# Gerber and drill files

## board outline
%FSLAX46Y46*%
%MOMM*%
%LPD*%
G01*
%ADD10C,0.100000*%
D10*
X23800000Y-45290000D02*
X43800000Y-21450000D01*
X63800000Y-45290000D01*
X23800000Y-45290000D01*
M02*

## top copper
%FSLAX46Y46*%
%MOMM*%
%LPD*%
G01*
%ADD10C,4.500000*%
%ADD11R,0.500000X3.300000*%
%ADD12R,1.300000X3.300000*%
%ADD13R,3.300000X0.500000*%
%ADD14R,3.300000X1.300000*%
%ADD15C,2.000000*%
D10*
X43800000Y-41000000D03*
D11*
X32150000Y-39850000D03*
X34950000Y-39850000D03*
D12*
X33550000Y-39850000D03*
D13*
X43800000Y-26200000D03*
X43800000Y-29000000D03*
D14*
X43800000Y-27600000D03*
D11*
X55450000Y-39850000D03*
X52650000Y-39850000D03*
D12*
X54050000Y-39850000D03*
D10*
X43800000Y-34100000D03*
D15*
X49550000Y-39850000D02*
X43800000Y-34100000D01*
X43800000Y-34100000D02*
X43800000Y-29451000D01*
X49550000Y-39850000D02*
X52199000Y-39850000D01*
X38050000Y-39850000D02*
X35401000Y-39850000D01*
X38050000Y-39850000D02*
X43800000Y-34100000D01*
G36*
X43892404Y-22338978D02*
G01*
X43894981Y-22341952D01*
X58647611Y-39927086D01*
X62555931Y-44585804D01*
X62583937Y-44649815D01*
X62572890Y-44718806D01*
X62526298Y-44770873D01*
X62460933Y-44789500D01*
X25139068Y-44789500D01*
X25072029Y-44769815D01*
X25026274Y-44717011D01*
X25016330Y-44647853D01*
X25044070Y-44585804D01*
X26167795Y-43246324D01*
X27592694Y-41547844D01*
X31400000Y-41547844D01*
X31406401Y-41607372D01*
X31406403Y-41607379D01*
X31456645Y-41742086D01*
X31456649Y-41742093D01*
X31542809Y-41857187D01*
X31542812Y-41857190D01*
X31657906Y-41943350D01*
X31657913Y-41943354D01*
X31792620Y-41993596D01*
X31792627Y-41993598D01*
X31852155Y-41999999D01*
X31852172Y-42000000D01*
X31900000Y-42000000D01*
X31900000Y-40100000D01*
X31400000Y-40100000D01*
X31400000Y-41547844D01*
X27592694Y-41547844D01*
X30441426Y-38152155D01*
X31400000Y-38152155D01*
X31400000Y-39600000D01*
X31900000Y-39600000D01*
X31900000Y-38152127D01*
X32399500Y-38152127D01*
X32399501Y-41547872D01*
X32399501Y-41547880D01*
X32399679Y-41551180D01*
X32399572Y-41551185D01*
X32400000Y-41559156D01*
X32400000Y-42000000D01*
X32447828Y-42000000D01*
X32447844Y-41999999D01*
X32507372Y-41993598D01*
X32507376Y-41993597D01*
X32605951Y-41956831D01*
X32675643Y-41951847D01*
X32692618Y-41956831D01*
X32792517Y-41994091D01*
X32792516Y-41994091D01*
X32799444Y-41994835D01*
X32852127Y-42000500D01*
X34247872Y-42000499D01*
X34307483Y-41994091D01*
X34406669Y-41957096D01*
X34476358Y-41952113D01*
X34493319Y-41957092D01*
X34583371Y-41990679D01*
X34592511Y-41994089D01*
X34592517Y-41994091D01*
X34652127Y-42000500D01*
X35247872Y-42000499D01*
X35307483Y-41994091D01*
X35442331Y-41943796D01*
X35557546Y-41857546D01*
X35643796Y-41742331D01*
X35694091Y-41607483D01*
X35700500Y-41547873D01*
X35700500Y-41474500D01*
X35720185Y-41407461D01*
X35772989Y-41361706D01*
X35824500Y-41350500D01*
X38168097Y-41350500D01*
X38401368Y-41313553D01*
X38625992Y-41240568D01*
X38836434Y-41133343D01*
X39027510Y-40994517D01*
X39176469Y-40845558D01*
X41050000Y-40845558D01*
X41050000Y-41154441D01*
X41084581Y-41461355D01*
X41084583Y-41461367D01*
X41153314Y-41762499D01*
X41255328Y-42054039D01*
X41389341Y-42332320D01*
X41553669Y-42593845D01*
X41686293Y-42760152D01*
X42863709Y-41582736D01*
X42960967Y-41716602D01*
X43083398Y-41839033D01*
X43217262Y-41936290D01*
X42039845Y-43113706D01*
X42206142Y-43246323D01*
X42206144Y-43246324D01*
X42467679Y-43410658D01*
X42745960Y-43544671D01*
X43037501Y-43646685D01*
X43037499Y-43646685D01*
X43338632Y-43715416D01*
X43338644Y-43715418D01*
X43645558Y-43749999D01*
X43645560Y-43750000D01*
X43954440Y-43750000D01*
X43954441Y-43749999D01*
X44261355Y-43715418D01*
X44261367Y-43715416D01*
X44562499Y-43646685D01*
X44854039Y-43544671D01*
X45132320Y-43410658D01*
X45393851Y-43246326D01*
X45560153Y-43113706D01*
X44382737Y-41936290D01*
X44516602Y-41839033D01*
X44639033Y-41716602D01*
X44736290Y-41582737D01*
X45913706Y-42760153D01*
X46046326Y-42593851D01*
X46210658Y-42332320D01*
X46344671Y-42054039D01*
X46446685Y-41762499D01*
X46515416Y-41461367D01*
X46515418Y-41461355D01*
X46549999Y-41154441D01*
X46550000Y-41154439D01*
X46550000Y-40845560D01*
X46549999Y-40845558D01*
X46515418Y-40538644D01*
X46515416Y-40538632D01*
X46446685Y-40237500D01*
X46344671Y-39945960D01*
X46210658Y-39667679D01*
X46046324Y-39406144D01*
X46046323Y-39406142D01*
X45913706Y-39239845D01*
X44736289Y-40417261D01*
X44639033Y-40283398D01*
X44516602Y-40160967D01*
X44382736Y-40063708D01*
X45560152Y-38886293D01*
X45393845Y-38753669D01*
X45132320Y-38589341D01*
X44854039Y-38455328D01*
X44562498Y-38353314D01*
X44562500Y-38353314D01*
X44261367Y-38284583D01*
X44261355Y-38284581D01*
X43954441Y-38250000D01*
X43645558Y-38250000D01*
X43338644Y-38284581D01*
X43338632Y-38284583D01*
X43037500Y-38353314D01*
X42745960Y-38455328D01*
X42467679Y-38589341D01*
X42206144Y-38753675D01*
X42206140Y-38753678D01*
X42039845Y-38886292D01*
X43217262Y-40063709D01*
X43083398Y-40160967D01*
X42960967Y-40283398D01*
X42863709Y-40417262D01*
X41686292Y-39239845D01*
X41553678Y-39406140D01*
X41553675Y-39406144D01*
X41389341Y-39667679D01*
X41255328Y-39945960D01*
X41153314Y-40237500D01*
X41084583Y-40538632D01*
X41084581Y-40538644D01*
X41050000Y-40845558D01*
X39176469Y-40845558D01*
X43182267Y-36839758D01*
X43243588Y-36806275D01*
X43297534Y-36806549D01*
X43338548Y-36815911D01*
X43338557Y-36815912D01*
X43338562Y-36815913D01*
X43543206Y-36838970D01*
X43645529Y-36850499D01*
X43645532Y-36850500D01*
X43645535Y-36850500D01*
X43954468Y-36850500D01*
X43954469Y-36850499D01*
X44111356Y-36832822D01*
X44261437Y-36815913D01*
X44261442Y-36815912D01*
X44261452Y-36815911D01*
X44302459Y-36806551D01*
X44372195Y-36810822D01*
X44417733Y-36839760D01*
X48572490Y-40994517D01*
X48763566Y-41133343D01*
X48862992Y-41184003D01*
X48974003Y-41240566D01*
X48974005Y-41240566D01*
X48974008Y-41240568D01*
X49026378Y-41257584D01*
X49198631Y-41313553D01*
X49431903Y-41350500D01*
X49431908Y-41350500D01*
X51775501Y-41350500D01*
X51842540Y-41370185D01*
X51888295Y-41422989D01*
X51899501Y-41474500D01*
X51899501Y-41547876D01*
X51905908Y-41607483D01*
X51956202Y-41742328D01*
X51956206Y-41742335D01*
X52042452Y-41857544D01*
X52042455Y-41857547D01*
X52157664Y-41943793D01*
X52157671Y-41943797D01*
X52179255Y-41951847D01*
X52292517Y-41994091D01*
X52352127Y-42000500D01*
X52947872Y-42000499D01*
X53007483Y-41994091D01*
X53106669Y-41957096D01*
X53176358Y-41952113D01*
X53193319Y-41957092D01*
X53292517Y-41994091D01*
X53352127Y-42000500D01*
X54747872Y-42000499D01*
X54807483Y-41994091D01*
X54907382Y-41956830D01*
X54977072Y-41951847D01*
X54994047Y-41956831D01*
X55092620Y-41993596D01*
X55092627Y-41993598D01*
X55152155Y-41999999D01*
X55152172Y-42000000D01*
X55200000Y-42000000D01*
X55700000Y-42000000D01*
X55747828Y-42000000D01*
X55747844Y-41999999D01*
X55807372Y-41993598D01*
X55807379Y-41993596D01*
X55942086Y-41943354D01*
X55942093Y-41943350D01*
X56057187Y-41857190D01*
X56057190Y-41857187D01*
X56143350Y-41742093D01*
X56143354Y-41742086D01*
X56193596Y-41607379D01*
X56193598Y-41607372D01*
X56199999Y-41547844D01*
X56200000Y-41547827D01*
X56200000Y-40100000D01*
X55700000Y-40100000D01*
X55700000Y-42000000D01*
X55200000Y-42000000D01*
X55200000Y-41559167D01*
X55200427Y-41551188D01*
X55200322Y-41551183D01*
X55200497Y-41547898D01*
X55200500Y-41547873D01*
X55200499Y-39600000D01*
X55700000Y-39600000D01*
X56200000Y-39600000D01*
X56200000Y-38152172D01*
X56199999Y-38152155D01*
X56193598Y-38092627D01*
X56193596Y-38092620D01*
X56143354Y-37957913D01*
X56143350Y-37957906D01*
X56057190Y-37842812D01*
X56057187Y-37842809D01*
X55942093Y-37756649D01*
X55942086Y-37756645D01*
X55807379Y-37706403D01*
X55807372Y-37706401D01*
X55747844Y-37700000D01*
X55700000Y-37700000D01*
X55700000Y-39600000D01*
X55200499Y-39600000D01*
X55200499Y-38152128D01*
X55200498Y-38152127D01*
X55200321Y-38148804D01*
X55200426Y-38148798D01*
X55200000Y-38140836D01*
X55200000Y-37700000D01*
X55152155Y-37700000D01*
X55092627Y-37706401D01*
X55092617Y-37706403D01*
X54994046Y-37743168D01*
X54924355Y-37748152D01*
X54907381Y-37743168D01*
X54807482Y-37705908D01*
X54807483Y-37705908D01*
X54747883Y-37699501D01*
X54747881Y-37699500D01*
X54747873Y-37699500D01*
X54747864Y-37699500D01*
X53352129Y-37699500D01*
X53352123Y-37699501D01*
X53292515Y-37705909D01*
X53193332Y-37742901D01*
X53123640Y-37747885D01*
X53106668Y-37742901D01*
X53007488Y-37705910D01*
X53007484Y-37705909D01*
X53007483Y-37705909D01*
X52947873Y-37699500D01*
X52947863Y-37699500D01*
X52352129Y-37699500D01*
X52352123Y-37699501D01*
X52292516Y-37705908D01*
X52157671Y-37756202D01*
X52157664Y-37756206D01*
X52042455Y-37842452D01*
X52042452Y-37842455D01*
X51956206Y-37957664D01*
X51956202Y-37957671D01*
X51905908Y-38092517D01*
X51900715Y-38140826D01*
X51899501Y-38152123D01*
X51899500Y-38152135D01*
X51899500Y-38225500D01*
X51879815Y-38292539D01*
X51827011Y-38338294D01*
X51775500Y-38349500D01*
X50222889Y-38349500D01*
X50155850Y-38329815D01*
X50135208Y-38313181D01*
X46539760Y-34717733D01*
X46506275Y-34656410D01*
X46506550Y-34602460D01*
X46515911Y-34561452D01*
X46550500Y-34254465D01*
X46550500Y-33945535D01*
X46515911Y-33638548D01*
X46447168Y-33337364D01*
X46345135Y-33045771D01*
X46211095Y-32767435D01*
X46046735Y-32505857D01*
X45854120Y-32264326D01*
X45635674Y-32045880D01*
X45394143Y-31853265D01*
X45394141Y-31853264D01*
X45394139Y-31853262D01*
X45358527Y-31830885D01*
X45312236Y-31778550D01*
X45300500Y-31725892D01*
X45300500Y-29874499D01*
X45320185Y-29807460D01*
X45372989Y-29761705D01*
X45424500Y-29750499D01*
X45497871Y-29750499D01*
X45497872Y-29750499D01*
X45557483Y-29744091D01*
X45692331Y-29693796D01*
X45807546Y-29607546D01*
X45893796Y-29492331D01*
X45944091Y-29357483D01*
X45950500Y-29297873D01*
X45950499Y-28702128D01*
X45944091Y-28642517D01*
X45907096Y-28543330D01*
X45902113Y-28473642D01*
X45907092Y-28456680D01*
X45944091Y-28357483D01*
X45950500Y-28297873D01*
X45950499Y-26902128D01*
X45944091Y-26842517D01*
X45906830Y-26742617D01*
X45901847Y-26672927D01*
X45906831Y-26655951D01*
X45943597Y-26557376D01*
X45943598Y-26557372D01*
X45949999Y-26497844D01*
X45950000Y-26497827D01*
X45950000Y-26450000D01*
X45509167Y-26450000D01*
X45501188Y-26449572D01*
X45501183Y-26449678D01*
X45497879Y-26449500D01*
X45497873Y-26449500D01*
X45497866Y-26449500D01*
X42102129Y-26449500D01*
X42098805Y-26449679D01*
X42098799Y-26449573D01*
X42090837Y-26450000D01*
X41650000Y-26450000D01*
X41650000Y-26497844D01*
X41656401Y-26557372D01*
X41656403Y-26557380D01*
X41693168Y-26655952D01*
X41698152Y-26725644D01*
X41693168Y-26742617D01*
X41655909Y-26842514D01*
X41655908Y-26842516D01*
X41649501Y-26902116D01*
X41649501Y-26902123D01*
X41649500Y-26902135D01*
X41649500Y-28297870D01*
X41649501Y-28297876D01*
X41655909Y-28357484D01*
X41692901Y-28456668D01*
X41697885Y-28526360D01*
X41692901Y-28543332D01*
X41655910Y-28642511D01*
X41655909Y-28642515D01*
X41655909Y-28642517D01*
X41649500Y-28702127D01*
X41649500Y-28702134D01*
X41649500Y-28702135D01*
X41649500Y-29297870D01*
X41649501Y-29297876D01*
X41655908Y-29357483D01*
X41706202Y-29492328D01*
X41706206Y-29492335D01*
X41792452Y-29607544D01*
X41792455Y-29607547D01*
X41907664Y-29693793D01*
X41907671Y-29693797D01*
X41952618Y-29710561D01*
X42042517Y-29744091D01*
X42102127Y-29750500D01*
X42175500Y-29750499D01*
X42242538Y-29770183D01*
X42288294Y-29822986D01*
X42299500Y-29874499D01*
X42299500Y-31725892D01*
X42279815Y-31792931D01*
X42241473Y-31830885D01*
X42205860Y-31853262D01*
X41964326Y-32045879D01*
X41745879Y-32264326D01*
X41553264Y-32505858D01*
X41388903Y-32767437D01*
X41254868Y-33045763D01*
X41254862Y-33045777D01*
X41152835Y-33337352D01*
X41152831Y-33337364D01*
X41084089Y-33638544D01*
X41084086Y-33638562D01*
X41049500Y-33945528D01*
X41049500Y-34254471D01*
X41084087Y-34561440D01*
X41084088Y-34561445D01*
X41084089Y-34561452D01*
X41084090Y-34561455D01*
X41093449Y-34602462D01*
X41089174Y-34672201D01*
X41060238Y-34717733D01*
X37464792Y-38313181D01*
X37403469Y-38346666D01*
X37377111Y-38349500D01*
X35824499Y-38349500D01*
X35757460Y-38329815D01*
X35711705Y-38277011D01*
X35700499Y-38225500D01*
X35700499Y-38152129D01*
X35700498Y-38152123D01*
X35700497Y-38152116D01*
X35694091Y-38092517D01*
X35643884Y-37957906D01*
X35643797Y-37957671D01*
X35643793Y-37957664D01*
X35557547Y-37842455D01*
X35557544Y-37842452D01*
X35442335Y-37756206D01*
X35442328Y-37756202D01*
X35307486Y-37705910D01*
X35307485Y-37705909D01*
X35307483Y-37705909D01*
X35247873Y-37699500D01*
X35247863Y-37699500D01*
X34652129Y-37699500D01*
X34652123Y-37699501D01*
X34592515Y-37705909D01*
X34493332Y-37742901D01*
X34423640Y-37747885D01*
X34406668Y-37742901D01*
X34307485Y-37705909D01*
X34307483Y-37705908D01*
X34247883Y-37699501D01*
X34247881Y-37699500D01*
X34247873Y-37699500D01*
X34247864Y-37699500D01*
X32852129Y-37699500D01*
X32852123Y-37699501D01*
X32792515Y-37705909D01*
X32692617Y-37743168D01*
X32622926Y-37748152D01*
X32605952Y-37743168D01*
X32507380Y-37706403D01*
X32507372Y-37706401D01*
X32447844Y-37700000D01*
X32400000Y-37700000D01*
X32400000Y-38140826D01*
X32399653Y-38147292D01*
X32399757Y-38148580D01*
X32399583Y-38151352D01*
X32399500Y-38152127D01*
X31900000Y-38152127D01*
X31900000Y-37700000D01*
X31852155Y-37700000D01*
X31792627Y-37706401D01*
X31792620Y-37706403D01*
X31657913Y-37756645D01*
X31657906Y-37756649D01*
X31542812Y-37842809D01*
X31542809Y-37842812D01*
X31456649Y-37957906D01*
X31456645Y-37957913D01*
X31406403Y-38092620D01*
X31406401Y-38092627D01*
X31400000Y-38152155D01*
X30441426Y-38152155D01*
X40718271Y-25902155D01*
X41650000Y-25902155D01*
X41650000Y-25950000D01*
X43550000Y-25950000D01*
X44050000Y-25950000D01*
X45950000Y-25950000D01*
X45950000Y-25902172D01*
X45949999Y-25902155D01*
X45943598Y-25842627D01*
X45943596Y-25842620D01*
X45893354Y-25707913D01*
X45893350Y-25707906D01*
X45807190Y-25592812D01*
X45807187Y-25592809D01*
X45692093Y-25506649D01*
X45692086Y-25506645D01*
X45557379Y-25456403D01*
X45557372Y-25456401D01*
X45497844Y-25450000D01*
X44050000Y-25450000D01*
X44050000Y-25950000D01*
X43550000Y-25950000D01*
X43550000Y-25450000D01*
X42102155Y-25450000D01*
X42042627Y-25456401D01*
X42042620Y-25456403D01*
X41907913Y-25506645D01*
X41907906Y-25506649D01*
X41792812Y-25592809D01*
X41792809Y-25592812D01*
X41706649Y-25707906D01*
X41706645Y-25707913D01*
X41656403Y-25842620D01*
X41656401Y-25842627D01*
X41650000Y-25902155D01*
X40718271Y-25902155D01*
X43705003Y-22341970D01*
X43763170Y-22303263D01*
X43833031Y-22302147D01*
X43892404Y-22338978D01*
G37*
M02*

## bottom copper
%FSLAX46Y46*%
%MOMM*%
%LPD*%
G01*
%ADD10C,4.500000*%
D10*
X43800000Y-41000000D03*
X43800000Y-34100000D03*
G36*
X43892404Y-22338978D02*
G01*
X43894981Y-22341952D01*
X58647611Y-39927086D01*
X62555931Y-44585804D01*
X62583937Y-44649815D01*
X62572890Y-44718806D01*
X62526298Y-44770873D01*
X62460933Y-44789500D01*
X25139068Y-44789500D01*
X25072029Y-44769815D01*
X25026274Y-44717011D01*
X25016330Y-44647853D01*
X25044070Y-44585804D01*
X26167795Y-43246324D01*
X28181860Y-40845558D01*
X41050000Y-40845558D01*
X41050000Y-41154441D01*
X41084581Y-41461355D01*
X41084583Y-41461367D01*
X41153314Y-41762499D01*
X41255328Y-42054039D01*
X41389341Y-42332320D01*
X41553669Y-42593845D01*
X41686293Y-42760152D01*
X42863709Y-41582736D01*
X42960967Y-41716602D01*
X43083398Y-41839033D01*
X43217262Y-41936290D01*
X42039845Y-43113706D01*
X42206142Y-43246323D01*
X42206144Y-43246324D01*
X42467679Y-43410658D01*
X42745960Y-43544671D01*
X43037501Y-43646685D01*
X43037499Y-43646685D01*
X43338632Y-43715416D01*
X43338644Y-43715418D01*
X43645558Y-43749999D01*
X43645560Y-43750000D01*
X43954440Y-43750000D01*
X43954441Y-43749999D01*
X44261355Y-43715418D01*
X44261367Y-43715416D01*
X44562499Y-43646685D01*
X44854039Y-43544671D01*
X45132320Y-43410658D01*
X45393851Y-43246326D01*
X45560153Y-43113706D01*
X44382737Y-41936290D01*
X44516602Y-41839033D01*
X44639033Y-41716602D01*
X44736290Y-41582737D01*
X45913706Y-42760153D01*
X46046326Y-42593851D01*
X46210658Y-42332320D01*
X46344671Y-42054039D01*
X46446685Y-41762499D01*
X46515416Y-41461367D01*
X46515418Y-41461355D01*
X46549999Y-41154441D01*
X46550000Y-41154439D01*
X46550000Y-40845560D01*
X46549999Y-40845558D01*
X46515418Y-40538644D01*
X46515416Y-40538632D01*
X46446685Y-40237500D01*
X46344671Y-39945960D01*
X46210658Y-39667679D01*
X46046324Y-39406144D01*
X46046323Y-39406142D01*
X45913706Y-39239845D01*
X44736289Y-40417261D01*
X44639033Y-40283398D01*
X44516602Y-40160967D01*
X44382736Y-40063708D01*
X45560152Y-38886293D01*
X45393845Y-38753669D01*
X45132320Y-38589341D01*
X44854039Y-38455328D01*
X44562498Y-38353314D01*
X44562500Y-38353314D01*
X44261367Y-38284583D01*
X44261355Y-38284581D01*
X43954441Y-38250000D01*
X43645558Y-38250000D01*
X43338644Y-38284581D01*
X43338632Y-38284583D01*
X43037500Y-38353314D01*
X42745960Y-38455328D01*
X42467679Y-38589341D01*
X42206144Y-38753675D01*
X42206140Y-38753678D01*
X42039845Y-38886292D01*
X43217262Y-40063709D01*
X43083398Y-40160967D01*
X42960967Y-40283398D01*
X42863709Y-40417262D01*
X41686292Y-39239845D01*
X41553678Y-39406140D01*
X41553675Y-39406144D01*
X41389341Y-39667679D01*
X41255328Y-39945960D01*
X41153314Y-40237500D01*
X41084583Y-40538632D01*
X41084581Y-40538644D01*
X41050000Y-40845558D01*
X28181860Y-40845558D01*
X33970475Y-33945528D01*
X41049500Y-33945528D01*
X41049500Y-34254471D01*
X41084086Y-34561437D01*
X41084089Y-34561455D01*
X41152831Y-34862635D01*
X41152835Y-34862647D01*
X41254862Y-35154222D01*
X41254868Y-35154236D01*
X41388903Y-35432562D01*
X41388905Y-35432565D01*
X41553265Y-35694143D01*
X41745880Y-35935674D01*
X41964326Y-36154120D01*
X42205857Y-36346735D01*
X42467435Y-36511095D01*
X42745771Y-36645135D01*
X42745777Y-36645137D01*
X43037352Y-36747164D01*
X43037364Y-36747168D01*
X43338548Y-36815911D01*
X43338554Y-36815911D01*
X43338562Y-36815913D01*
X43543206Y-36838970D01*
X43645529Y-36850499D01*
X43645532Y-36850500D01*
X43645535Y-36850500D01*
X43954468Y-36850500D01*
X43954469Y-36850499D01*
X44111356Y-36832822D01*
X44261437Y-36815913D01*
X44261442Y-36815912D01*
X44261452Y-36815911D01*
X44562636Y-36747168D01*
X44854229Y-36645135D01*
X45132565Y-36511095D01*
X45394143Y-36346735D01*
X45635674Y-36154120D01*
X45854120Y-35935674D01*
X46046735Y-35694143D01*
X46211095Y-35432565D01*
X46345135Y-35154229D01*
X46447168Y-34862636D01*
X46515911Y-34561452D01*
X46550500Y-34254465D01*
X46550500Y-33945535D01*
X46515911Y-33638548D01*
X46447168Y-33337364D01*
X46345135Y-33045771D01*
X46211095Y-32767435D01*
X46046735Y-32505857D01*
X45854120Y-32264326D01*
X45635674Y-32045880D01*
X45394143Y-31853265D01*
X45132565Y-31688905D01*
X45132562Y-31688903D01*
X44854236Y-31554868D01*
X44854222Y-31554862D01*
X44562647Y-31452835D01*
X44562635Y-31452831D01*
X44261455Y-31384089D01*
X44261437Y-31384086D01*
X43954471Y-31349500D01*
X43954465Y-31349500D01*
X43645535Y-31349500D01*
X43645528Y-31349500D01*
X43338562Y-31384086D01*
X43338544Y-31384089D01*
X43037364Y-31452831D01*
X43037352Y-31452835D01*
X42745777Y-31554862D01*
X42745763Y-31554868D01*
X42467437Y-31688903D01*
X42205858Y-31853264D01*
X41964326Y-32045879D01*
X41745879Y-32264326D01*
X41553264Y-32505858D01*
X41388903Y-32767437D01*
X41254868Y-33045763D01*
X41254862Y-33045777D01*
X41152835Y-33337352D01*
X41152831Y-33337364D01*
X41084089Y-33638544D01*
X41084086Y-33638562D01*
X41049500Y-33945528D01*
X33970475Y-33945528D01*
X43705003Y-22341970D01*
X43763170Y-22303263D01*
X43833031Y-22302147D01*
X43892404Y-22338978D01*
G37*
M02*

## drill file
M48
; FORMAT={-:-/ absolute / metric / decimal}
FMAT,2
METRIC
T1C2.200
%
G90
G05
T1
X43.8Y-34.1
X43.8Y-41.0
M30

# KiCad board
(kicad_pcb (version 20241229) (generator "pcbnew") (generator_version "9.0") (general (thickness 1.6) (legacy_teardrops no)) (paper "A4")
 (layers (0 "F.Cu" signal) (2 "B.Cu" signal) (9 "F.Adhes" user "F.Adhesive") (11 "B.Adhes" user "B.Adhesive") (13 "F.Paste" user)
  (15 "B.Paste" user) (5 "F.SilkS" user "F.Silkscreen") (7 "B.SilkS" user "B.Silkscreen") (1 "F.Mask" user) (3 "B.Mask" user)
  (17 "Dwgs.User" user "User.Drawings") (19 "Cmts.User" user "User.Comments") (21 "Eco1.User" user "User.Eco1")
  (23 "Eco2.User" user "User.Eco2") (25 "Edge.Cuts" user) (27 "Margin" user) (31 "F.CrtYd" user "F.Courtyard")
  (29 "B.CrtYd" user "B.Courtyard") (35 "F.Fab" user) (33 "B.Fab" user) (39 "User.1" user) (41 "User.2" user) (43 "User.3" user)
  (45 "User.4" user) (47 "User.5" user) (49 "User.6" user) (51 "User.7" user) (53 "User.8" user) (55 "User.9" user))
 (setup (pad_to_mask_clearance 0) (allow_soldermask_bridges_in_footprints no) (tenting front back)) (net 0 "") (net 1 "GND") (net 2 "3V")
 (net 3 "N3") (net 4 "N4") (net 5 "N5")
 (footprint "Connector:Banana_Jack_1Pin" (layer "F.Cu") (at 43.8 41)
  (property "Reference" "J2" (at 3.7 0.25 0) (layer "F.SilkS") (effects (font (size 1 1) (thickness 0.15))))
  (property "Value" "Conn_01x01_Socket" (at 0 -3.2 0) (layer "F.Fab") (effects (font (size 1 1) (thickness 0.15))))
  (pad "1" thru_hole circle (at 0 0) (size 4.5 4.5) (drill 2.2) (layers "*.Cu" "*.Mask") (remove_unused_layers no) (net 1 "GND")))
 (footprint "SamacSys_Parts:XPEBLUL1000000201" (layer "F.Cu") (at 33.55 39.85)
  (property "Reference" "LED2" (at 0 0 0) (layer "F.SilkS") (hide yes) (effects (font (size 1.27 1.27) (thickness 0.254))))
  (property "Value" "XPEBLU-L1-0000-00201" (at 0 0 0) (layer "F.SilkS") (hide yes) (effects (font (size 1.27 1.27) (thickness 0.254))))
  (pad "1" smd rect (at -1.4 0) (size 0.5 3.3) (layers "F.Cu" "F.Mask" "F.Paste") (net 1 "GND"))
  (pad "2" smd rect (at 1.4 0) (size 0.5 3.3) (layers "F.Cu" "F.Mask" "F.Paste") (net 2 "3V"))
  (pad "3" smd rect (at 0 0) (size 1.3 3.3) (layers "F.Cu" "F.Mask" "F.Paste") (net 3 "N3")))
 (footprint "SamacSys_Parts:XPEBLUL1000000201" (layer "F.Cu") (at 43.8 27.6 -90)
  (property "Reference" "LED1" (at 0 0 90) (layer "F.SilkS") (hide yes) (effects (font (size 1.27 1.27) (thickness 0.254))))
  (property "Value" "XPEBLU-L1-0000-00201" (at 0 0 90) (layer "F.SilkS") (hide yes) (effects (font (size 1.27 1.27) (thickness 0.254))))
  (pad "1" smd rect (at -1.4 0 270) (size 0.5 3.3) (layers "F.Cu" "F.Mask" "F.Paste") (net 1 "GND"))
  (pad "2" smd rect (at 1.4 0 270) (size 0.5 3.3) (layers "F.Cu" "F.Mask" "F.Paste") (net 2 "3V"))
  (pad "3" smd rect (at 0 0 270) (size 1.3 3.3) (layers "F.Cu" "F.Mask" "F.Paste") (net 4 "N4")))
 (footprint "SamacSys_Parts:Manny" (layer "F.Cu") (at 50.85 40.35)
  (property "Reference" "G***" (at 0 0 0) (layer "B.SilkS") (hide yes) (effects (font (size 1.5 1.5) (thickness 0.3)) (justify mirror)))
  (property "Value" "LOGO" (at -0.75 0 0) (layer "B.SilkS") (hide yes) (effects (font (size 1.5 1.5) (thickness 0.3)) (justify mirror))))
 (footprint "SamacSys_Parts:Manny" (layer "F.Cu") (at 36.65 40.45)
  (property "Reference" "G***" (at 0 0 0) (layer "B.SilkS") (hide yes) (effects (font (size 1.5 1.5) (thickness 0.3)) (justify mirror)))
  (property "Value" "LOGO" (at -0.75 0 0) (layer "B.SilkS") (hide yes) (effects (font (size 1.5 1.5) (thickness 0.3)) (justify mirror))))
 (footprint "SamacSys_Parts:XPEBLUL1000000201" (layer "F.Cu") (at 54.05 39.85 180)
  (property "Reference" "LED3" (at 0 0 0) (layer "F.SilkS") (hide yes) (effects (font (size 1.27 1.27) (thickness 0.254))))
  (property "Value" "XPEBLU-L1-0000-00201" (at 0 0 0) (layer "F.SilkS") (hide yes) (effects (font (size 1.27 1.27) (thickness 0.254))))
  (pad "1" smd rect (at -1.4 0 180) (size 0.5 3.3) (layers "F.Cu" "F.Mask" "F.Paste") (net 1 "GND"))
  (pad "2" smd rect (at 1.4 0 180) (size 0.5 3.3) (layers "F.Cu" "F.Mask" "F.Paste") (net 2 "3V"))
  (pad "3" smd rect (at 0 0 180) (size 1.3 3.3) (layers "F.Cu" "F.Mask" "F.Paste") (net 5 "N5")))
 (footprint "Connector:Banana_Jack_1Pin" (layer "F.Cu") (at 43.8 34.1)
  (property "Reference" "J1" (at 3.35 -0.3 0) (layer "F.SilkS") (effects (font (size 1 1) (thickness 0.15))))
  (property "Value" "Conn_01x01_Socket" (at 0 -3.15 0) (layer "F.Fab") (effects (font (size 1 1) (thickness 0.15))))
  (pad "1" thru_hole circle (at 0 0) (size 4.5 4.5) (drill 2.2) (layers "*.Cu" "*.Mask") (remove_unused_layers no) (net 2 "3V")))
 (gr_poly (pts (xy 23.8 45.29) (xy 43.8 21.45) (xy 63.8 45.29)) (stroke (width 0.1) (type solid)) (fill no) (layer "Edge.Cuts"))
 (segment (start 49.55 39.85) (end 43.8 34.1) (width 2) (layer "F.Cu") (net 2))
 (segment (start 43.8 34.1) (end 43.8 29.451) (width 2) (layer "F.Cu") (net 2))
 (segment (start 49.55 39.85) (end 52.199 39.85) (width 2) (layer "F.Cu") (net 2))
 (segment (start 38.05 39.85) (end 35.401 39.85) (width 2) (layer "F.Cu") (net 2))
 (segment (start 38.05 39.85) (end 43.8 34.1) (width 2) (layer "F.Cu") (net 2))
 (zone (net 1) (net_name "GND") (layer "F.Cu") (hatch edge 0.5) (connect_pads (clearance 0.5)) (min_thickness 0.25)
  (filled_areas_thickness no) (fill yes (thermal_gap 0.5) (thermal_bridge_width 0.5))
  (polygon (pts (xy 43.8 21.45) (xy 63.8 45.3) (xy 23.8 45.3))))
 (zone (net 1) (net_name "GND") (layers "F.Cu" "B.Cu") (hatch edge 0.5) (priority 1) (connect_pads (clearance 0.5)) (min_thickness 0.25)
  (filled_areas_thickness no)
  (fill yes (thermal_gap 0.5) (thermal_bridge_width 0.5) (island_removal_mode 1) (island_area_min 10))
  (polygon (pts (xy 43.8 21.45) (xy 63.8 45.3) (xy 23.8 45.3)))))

